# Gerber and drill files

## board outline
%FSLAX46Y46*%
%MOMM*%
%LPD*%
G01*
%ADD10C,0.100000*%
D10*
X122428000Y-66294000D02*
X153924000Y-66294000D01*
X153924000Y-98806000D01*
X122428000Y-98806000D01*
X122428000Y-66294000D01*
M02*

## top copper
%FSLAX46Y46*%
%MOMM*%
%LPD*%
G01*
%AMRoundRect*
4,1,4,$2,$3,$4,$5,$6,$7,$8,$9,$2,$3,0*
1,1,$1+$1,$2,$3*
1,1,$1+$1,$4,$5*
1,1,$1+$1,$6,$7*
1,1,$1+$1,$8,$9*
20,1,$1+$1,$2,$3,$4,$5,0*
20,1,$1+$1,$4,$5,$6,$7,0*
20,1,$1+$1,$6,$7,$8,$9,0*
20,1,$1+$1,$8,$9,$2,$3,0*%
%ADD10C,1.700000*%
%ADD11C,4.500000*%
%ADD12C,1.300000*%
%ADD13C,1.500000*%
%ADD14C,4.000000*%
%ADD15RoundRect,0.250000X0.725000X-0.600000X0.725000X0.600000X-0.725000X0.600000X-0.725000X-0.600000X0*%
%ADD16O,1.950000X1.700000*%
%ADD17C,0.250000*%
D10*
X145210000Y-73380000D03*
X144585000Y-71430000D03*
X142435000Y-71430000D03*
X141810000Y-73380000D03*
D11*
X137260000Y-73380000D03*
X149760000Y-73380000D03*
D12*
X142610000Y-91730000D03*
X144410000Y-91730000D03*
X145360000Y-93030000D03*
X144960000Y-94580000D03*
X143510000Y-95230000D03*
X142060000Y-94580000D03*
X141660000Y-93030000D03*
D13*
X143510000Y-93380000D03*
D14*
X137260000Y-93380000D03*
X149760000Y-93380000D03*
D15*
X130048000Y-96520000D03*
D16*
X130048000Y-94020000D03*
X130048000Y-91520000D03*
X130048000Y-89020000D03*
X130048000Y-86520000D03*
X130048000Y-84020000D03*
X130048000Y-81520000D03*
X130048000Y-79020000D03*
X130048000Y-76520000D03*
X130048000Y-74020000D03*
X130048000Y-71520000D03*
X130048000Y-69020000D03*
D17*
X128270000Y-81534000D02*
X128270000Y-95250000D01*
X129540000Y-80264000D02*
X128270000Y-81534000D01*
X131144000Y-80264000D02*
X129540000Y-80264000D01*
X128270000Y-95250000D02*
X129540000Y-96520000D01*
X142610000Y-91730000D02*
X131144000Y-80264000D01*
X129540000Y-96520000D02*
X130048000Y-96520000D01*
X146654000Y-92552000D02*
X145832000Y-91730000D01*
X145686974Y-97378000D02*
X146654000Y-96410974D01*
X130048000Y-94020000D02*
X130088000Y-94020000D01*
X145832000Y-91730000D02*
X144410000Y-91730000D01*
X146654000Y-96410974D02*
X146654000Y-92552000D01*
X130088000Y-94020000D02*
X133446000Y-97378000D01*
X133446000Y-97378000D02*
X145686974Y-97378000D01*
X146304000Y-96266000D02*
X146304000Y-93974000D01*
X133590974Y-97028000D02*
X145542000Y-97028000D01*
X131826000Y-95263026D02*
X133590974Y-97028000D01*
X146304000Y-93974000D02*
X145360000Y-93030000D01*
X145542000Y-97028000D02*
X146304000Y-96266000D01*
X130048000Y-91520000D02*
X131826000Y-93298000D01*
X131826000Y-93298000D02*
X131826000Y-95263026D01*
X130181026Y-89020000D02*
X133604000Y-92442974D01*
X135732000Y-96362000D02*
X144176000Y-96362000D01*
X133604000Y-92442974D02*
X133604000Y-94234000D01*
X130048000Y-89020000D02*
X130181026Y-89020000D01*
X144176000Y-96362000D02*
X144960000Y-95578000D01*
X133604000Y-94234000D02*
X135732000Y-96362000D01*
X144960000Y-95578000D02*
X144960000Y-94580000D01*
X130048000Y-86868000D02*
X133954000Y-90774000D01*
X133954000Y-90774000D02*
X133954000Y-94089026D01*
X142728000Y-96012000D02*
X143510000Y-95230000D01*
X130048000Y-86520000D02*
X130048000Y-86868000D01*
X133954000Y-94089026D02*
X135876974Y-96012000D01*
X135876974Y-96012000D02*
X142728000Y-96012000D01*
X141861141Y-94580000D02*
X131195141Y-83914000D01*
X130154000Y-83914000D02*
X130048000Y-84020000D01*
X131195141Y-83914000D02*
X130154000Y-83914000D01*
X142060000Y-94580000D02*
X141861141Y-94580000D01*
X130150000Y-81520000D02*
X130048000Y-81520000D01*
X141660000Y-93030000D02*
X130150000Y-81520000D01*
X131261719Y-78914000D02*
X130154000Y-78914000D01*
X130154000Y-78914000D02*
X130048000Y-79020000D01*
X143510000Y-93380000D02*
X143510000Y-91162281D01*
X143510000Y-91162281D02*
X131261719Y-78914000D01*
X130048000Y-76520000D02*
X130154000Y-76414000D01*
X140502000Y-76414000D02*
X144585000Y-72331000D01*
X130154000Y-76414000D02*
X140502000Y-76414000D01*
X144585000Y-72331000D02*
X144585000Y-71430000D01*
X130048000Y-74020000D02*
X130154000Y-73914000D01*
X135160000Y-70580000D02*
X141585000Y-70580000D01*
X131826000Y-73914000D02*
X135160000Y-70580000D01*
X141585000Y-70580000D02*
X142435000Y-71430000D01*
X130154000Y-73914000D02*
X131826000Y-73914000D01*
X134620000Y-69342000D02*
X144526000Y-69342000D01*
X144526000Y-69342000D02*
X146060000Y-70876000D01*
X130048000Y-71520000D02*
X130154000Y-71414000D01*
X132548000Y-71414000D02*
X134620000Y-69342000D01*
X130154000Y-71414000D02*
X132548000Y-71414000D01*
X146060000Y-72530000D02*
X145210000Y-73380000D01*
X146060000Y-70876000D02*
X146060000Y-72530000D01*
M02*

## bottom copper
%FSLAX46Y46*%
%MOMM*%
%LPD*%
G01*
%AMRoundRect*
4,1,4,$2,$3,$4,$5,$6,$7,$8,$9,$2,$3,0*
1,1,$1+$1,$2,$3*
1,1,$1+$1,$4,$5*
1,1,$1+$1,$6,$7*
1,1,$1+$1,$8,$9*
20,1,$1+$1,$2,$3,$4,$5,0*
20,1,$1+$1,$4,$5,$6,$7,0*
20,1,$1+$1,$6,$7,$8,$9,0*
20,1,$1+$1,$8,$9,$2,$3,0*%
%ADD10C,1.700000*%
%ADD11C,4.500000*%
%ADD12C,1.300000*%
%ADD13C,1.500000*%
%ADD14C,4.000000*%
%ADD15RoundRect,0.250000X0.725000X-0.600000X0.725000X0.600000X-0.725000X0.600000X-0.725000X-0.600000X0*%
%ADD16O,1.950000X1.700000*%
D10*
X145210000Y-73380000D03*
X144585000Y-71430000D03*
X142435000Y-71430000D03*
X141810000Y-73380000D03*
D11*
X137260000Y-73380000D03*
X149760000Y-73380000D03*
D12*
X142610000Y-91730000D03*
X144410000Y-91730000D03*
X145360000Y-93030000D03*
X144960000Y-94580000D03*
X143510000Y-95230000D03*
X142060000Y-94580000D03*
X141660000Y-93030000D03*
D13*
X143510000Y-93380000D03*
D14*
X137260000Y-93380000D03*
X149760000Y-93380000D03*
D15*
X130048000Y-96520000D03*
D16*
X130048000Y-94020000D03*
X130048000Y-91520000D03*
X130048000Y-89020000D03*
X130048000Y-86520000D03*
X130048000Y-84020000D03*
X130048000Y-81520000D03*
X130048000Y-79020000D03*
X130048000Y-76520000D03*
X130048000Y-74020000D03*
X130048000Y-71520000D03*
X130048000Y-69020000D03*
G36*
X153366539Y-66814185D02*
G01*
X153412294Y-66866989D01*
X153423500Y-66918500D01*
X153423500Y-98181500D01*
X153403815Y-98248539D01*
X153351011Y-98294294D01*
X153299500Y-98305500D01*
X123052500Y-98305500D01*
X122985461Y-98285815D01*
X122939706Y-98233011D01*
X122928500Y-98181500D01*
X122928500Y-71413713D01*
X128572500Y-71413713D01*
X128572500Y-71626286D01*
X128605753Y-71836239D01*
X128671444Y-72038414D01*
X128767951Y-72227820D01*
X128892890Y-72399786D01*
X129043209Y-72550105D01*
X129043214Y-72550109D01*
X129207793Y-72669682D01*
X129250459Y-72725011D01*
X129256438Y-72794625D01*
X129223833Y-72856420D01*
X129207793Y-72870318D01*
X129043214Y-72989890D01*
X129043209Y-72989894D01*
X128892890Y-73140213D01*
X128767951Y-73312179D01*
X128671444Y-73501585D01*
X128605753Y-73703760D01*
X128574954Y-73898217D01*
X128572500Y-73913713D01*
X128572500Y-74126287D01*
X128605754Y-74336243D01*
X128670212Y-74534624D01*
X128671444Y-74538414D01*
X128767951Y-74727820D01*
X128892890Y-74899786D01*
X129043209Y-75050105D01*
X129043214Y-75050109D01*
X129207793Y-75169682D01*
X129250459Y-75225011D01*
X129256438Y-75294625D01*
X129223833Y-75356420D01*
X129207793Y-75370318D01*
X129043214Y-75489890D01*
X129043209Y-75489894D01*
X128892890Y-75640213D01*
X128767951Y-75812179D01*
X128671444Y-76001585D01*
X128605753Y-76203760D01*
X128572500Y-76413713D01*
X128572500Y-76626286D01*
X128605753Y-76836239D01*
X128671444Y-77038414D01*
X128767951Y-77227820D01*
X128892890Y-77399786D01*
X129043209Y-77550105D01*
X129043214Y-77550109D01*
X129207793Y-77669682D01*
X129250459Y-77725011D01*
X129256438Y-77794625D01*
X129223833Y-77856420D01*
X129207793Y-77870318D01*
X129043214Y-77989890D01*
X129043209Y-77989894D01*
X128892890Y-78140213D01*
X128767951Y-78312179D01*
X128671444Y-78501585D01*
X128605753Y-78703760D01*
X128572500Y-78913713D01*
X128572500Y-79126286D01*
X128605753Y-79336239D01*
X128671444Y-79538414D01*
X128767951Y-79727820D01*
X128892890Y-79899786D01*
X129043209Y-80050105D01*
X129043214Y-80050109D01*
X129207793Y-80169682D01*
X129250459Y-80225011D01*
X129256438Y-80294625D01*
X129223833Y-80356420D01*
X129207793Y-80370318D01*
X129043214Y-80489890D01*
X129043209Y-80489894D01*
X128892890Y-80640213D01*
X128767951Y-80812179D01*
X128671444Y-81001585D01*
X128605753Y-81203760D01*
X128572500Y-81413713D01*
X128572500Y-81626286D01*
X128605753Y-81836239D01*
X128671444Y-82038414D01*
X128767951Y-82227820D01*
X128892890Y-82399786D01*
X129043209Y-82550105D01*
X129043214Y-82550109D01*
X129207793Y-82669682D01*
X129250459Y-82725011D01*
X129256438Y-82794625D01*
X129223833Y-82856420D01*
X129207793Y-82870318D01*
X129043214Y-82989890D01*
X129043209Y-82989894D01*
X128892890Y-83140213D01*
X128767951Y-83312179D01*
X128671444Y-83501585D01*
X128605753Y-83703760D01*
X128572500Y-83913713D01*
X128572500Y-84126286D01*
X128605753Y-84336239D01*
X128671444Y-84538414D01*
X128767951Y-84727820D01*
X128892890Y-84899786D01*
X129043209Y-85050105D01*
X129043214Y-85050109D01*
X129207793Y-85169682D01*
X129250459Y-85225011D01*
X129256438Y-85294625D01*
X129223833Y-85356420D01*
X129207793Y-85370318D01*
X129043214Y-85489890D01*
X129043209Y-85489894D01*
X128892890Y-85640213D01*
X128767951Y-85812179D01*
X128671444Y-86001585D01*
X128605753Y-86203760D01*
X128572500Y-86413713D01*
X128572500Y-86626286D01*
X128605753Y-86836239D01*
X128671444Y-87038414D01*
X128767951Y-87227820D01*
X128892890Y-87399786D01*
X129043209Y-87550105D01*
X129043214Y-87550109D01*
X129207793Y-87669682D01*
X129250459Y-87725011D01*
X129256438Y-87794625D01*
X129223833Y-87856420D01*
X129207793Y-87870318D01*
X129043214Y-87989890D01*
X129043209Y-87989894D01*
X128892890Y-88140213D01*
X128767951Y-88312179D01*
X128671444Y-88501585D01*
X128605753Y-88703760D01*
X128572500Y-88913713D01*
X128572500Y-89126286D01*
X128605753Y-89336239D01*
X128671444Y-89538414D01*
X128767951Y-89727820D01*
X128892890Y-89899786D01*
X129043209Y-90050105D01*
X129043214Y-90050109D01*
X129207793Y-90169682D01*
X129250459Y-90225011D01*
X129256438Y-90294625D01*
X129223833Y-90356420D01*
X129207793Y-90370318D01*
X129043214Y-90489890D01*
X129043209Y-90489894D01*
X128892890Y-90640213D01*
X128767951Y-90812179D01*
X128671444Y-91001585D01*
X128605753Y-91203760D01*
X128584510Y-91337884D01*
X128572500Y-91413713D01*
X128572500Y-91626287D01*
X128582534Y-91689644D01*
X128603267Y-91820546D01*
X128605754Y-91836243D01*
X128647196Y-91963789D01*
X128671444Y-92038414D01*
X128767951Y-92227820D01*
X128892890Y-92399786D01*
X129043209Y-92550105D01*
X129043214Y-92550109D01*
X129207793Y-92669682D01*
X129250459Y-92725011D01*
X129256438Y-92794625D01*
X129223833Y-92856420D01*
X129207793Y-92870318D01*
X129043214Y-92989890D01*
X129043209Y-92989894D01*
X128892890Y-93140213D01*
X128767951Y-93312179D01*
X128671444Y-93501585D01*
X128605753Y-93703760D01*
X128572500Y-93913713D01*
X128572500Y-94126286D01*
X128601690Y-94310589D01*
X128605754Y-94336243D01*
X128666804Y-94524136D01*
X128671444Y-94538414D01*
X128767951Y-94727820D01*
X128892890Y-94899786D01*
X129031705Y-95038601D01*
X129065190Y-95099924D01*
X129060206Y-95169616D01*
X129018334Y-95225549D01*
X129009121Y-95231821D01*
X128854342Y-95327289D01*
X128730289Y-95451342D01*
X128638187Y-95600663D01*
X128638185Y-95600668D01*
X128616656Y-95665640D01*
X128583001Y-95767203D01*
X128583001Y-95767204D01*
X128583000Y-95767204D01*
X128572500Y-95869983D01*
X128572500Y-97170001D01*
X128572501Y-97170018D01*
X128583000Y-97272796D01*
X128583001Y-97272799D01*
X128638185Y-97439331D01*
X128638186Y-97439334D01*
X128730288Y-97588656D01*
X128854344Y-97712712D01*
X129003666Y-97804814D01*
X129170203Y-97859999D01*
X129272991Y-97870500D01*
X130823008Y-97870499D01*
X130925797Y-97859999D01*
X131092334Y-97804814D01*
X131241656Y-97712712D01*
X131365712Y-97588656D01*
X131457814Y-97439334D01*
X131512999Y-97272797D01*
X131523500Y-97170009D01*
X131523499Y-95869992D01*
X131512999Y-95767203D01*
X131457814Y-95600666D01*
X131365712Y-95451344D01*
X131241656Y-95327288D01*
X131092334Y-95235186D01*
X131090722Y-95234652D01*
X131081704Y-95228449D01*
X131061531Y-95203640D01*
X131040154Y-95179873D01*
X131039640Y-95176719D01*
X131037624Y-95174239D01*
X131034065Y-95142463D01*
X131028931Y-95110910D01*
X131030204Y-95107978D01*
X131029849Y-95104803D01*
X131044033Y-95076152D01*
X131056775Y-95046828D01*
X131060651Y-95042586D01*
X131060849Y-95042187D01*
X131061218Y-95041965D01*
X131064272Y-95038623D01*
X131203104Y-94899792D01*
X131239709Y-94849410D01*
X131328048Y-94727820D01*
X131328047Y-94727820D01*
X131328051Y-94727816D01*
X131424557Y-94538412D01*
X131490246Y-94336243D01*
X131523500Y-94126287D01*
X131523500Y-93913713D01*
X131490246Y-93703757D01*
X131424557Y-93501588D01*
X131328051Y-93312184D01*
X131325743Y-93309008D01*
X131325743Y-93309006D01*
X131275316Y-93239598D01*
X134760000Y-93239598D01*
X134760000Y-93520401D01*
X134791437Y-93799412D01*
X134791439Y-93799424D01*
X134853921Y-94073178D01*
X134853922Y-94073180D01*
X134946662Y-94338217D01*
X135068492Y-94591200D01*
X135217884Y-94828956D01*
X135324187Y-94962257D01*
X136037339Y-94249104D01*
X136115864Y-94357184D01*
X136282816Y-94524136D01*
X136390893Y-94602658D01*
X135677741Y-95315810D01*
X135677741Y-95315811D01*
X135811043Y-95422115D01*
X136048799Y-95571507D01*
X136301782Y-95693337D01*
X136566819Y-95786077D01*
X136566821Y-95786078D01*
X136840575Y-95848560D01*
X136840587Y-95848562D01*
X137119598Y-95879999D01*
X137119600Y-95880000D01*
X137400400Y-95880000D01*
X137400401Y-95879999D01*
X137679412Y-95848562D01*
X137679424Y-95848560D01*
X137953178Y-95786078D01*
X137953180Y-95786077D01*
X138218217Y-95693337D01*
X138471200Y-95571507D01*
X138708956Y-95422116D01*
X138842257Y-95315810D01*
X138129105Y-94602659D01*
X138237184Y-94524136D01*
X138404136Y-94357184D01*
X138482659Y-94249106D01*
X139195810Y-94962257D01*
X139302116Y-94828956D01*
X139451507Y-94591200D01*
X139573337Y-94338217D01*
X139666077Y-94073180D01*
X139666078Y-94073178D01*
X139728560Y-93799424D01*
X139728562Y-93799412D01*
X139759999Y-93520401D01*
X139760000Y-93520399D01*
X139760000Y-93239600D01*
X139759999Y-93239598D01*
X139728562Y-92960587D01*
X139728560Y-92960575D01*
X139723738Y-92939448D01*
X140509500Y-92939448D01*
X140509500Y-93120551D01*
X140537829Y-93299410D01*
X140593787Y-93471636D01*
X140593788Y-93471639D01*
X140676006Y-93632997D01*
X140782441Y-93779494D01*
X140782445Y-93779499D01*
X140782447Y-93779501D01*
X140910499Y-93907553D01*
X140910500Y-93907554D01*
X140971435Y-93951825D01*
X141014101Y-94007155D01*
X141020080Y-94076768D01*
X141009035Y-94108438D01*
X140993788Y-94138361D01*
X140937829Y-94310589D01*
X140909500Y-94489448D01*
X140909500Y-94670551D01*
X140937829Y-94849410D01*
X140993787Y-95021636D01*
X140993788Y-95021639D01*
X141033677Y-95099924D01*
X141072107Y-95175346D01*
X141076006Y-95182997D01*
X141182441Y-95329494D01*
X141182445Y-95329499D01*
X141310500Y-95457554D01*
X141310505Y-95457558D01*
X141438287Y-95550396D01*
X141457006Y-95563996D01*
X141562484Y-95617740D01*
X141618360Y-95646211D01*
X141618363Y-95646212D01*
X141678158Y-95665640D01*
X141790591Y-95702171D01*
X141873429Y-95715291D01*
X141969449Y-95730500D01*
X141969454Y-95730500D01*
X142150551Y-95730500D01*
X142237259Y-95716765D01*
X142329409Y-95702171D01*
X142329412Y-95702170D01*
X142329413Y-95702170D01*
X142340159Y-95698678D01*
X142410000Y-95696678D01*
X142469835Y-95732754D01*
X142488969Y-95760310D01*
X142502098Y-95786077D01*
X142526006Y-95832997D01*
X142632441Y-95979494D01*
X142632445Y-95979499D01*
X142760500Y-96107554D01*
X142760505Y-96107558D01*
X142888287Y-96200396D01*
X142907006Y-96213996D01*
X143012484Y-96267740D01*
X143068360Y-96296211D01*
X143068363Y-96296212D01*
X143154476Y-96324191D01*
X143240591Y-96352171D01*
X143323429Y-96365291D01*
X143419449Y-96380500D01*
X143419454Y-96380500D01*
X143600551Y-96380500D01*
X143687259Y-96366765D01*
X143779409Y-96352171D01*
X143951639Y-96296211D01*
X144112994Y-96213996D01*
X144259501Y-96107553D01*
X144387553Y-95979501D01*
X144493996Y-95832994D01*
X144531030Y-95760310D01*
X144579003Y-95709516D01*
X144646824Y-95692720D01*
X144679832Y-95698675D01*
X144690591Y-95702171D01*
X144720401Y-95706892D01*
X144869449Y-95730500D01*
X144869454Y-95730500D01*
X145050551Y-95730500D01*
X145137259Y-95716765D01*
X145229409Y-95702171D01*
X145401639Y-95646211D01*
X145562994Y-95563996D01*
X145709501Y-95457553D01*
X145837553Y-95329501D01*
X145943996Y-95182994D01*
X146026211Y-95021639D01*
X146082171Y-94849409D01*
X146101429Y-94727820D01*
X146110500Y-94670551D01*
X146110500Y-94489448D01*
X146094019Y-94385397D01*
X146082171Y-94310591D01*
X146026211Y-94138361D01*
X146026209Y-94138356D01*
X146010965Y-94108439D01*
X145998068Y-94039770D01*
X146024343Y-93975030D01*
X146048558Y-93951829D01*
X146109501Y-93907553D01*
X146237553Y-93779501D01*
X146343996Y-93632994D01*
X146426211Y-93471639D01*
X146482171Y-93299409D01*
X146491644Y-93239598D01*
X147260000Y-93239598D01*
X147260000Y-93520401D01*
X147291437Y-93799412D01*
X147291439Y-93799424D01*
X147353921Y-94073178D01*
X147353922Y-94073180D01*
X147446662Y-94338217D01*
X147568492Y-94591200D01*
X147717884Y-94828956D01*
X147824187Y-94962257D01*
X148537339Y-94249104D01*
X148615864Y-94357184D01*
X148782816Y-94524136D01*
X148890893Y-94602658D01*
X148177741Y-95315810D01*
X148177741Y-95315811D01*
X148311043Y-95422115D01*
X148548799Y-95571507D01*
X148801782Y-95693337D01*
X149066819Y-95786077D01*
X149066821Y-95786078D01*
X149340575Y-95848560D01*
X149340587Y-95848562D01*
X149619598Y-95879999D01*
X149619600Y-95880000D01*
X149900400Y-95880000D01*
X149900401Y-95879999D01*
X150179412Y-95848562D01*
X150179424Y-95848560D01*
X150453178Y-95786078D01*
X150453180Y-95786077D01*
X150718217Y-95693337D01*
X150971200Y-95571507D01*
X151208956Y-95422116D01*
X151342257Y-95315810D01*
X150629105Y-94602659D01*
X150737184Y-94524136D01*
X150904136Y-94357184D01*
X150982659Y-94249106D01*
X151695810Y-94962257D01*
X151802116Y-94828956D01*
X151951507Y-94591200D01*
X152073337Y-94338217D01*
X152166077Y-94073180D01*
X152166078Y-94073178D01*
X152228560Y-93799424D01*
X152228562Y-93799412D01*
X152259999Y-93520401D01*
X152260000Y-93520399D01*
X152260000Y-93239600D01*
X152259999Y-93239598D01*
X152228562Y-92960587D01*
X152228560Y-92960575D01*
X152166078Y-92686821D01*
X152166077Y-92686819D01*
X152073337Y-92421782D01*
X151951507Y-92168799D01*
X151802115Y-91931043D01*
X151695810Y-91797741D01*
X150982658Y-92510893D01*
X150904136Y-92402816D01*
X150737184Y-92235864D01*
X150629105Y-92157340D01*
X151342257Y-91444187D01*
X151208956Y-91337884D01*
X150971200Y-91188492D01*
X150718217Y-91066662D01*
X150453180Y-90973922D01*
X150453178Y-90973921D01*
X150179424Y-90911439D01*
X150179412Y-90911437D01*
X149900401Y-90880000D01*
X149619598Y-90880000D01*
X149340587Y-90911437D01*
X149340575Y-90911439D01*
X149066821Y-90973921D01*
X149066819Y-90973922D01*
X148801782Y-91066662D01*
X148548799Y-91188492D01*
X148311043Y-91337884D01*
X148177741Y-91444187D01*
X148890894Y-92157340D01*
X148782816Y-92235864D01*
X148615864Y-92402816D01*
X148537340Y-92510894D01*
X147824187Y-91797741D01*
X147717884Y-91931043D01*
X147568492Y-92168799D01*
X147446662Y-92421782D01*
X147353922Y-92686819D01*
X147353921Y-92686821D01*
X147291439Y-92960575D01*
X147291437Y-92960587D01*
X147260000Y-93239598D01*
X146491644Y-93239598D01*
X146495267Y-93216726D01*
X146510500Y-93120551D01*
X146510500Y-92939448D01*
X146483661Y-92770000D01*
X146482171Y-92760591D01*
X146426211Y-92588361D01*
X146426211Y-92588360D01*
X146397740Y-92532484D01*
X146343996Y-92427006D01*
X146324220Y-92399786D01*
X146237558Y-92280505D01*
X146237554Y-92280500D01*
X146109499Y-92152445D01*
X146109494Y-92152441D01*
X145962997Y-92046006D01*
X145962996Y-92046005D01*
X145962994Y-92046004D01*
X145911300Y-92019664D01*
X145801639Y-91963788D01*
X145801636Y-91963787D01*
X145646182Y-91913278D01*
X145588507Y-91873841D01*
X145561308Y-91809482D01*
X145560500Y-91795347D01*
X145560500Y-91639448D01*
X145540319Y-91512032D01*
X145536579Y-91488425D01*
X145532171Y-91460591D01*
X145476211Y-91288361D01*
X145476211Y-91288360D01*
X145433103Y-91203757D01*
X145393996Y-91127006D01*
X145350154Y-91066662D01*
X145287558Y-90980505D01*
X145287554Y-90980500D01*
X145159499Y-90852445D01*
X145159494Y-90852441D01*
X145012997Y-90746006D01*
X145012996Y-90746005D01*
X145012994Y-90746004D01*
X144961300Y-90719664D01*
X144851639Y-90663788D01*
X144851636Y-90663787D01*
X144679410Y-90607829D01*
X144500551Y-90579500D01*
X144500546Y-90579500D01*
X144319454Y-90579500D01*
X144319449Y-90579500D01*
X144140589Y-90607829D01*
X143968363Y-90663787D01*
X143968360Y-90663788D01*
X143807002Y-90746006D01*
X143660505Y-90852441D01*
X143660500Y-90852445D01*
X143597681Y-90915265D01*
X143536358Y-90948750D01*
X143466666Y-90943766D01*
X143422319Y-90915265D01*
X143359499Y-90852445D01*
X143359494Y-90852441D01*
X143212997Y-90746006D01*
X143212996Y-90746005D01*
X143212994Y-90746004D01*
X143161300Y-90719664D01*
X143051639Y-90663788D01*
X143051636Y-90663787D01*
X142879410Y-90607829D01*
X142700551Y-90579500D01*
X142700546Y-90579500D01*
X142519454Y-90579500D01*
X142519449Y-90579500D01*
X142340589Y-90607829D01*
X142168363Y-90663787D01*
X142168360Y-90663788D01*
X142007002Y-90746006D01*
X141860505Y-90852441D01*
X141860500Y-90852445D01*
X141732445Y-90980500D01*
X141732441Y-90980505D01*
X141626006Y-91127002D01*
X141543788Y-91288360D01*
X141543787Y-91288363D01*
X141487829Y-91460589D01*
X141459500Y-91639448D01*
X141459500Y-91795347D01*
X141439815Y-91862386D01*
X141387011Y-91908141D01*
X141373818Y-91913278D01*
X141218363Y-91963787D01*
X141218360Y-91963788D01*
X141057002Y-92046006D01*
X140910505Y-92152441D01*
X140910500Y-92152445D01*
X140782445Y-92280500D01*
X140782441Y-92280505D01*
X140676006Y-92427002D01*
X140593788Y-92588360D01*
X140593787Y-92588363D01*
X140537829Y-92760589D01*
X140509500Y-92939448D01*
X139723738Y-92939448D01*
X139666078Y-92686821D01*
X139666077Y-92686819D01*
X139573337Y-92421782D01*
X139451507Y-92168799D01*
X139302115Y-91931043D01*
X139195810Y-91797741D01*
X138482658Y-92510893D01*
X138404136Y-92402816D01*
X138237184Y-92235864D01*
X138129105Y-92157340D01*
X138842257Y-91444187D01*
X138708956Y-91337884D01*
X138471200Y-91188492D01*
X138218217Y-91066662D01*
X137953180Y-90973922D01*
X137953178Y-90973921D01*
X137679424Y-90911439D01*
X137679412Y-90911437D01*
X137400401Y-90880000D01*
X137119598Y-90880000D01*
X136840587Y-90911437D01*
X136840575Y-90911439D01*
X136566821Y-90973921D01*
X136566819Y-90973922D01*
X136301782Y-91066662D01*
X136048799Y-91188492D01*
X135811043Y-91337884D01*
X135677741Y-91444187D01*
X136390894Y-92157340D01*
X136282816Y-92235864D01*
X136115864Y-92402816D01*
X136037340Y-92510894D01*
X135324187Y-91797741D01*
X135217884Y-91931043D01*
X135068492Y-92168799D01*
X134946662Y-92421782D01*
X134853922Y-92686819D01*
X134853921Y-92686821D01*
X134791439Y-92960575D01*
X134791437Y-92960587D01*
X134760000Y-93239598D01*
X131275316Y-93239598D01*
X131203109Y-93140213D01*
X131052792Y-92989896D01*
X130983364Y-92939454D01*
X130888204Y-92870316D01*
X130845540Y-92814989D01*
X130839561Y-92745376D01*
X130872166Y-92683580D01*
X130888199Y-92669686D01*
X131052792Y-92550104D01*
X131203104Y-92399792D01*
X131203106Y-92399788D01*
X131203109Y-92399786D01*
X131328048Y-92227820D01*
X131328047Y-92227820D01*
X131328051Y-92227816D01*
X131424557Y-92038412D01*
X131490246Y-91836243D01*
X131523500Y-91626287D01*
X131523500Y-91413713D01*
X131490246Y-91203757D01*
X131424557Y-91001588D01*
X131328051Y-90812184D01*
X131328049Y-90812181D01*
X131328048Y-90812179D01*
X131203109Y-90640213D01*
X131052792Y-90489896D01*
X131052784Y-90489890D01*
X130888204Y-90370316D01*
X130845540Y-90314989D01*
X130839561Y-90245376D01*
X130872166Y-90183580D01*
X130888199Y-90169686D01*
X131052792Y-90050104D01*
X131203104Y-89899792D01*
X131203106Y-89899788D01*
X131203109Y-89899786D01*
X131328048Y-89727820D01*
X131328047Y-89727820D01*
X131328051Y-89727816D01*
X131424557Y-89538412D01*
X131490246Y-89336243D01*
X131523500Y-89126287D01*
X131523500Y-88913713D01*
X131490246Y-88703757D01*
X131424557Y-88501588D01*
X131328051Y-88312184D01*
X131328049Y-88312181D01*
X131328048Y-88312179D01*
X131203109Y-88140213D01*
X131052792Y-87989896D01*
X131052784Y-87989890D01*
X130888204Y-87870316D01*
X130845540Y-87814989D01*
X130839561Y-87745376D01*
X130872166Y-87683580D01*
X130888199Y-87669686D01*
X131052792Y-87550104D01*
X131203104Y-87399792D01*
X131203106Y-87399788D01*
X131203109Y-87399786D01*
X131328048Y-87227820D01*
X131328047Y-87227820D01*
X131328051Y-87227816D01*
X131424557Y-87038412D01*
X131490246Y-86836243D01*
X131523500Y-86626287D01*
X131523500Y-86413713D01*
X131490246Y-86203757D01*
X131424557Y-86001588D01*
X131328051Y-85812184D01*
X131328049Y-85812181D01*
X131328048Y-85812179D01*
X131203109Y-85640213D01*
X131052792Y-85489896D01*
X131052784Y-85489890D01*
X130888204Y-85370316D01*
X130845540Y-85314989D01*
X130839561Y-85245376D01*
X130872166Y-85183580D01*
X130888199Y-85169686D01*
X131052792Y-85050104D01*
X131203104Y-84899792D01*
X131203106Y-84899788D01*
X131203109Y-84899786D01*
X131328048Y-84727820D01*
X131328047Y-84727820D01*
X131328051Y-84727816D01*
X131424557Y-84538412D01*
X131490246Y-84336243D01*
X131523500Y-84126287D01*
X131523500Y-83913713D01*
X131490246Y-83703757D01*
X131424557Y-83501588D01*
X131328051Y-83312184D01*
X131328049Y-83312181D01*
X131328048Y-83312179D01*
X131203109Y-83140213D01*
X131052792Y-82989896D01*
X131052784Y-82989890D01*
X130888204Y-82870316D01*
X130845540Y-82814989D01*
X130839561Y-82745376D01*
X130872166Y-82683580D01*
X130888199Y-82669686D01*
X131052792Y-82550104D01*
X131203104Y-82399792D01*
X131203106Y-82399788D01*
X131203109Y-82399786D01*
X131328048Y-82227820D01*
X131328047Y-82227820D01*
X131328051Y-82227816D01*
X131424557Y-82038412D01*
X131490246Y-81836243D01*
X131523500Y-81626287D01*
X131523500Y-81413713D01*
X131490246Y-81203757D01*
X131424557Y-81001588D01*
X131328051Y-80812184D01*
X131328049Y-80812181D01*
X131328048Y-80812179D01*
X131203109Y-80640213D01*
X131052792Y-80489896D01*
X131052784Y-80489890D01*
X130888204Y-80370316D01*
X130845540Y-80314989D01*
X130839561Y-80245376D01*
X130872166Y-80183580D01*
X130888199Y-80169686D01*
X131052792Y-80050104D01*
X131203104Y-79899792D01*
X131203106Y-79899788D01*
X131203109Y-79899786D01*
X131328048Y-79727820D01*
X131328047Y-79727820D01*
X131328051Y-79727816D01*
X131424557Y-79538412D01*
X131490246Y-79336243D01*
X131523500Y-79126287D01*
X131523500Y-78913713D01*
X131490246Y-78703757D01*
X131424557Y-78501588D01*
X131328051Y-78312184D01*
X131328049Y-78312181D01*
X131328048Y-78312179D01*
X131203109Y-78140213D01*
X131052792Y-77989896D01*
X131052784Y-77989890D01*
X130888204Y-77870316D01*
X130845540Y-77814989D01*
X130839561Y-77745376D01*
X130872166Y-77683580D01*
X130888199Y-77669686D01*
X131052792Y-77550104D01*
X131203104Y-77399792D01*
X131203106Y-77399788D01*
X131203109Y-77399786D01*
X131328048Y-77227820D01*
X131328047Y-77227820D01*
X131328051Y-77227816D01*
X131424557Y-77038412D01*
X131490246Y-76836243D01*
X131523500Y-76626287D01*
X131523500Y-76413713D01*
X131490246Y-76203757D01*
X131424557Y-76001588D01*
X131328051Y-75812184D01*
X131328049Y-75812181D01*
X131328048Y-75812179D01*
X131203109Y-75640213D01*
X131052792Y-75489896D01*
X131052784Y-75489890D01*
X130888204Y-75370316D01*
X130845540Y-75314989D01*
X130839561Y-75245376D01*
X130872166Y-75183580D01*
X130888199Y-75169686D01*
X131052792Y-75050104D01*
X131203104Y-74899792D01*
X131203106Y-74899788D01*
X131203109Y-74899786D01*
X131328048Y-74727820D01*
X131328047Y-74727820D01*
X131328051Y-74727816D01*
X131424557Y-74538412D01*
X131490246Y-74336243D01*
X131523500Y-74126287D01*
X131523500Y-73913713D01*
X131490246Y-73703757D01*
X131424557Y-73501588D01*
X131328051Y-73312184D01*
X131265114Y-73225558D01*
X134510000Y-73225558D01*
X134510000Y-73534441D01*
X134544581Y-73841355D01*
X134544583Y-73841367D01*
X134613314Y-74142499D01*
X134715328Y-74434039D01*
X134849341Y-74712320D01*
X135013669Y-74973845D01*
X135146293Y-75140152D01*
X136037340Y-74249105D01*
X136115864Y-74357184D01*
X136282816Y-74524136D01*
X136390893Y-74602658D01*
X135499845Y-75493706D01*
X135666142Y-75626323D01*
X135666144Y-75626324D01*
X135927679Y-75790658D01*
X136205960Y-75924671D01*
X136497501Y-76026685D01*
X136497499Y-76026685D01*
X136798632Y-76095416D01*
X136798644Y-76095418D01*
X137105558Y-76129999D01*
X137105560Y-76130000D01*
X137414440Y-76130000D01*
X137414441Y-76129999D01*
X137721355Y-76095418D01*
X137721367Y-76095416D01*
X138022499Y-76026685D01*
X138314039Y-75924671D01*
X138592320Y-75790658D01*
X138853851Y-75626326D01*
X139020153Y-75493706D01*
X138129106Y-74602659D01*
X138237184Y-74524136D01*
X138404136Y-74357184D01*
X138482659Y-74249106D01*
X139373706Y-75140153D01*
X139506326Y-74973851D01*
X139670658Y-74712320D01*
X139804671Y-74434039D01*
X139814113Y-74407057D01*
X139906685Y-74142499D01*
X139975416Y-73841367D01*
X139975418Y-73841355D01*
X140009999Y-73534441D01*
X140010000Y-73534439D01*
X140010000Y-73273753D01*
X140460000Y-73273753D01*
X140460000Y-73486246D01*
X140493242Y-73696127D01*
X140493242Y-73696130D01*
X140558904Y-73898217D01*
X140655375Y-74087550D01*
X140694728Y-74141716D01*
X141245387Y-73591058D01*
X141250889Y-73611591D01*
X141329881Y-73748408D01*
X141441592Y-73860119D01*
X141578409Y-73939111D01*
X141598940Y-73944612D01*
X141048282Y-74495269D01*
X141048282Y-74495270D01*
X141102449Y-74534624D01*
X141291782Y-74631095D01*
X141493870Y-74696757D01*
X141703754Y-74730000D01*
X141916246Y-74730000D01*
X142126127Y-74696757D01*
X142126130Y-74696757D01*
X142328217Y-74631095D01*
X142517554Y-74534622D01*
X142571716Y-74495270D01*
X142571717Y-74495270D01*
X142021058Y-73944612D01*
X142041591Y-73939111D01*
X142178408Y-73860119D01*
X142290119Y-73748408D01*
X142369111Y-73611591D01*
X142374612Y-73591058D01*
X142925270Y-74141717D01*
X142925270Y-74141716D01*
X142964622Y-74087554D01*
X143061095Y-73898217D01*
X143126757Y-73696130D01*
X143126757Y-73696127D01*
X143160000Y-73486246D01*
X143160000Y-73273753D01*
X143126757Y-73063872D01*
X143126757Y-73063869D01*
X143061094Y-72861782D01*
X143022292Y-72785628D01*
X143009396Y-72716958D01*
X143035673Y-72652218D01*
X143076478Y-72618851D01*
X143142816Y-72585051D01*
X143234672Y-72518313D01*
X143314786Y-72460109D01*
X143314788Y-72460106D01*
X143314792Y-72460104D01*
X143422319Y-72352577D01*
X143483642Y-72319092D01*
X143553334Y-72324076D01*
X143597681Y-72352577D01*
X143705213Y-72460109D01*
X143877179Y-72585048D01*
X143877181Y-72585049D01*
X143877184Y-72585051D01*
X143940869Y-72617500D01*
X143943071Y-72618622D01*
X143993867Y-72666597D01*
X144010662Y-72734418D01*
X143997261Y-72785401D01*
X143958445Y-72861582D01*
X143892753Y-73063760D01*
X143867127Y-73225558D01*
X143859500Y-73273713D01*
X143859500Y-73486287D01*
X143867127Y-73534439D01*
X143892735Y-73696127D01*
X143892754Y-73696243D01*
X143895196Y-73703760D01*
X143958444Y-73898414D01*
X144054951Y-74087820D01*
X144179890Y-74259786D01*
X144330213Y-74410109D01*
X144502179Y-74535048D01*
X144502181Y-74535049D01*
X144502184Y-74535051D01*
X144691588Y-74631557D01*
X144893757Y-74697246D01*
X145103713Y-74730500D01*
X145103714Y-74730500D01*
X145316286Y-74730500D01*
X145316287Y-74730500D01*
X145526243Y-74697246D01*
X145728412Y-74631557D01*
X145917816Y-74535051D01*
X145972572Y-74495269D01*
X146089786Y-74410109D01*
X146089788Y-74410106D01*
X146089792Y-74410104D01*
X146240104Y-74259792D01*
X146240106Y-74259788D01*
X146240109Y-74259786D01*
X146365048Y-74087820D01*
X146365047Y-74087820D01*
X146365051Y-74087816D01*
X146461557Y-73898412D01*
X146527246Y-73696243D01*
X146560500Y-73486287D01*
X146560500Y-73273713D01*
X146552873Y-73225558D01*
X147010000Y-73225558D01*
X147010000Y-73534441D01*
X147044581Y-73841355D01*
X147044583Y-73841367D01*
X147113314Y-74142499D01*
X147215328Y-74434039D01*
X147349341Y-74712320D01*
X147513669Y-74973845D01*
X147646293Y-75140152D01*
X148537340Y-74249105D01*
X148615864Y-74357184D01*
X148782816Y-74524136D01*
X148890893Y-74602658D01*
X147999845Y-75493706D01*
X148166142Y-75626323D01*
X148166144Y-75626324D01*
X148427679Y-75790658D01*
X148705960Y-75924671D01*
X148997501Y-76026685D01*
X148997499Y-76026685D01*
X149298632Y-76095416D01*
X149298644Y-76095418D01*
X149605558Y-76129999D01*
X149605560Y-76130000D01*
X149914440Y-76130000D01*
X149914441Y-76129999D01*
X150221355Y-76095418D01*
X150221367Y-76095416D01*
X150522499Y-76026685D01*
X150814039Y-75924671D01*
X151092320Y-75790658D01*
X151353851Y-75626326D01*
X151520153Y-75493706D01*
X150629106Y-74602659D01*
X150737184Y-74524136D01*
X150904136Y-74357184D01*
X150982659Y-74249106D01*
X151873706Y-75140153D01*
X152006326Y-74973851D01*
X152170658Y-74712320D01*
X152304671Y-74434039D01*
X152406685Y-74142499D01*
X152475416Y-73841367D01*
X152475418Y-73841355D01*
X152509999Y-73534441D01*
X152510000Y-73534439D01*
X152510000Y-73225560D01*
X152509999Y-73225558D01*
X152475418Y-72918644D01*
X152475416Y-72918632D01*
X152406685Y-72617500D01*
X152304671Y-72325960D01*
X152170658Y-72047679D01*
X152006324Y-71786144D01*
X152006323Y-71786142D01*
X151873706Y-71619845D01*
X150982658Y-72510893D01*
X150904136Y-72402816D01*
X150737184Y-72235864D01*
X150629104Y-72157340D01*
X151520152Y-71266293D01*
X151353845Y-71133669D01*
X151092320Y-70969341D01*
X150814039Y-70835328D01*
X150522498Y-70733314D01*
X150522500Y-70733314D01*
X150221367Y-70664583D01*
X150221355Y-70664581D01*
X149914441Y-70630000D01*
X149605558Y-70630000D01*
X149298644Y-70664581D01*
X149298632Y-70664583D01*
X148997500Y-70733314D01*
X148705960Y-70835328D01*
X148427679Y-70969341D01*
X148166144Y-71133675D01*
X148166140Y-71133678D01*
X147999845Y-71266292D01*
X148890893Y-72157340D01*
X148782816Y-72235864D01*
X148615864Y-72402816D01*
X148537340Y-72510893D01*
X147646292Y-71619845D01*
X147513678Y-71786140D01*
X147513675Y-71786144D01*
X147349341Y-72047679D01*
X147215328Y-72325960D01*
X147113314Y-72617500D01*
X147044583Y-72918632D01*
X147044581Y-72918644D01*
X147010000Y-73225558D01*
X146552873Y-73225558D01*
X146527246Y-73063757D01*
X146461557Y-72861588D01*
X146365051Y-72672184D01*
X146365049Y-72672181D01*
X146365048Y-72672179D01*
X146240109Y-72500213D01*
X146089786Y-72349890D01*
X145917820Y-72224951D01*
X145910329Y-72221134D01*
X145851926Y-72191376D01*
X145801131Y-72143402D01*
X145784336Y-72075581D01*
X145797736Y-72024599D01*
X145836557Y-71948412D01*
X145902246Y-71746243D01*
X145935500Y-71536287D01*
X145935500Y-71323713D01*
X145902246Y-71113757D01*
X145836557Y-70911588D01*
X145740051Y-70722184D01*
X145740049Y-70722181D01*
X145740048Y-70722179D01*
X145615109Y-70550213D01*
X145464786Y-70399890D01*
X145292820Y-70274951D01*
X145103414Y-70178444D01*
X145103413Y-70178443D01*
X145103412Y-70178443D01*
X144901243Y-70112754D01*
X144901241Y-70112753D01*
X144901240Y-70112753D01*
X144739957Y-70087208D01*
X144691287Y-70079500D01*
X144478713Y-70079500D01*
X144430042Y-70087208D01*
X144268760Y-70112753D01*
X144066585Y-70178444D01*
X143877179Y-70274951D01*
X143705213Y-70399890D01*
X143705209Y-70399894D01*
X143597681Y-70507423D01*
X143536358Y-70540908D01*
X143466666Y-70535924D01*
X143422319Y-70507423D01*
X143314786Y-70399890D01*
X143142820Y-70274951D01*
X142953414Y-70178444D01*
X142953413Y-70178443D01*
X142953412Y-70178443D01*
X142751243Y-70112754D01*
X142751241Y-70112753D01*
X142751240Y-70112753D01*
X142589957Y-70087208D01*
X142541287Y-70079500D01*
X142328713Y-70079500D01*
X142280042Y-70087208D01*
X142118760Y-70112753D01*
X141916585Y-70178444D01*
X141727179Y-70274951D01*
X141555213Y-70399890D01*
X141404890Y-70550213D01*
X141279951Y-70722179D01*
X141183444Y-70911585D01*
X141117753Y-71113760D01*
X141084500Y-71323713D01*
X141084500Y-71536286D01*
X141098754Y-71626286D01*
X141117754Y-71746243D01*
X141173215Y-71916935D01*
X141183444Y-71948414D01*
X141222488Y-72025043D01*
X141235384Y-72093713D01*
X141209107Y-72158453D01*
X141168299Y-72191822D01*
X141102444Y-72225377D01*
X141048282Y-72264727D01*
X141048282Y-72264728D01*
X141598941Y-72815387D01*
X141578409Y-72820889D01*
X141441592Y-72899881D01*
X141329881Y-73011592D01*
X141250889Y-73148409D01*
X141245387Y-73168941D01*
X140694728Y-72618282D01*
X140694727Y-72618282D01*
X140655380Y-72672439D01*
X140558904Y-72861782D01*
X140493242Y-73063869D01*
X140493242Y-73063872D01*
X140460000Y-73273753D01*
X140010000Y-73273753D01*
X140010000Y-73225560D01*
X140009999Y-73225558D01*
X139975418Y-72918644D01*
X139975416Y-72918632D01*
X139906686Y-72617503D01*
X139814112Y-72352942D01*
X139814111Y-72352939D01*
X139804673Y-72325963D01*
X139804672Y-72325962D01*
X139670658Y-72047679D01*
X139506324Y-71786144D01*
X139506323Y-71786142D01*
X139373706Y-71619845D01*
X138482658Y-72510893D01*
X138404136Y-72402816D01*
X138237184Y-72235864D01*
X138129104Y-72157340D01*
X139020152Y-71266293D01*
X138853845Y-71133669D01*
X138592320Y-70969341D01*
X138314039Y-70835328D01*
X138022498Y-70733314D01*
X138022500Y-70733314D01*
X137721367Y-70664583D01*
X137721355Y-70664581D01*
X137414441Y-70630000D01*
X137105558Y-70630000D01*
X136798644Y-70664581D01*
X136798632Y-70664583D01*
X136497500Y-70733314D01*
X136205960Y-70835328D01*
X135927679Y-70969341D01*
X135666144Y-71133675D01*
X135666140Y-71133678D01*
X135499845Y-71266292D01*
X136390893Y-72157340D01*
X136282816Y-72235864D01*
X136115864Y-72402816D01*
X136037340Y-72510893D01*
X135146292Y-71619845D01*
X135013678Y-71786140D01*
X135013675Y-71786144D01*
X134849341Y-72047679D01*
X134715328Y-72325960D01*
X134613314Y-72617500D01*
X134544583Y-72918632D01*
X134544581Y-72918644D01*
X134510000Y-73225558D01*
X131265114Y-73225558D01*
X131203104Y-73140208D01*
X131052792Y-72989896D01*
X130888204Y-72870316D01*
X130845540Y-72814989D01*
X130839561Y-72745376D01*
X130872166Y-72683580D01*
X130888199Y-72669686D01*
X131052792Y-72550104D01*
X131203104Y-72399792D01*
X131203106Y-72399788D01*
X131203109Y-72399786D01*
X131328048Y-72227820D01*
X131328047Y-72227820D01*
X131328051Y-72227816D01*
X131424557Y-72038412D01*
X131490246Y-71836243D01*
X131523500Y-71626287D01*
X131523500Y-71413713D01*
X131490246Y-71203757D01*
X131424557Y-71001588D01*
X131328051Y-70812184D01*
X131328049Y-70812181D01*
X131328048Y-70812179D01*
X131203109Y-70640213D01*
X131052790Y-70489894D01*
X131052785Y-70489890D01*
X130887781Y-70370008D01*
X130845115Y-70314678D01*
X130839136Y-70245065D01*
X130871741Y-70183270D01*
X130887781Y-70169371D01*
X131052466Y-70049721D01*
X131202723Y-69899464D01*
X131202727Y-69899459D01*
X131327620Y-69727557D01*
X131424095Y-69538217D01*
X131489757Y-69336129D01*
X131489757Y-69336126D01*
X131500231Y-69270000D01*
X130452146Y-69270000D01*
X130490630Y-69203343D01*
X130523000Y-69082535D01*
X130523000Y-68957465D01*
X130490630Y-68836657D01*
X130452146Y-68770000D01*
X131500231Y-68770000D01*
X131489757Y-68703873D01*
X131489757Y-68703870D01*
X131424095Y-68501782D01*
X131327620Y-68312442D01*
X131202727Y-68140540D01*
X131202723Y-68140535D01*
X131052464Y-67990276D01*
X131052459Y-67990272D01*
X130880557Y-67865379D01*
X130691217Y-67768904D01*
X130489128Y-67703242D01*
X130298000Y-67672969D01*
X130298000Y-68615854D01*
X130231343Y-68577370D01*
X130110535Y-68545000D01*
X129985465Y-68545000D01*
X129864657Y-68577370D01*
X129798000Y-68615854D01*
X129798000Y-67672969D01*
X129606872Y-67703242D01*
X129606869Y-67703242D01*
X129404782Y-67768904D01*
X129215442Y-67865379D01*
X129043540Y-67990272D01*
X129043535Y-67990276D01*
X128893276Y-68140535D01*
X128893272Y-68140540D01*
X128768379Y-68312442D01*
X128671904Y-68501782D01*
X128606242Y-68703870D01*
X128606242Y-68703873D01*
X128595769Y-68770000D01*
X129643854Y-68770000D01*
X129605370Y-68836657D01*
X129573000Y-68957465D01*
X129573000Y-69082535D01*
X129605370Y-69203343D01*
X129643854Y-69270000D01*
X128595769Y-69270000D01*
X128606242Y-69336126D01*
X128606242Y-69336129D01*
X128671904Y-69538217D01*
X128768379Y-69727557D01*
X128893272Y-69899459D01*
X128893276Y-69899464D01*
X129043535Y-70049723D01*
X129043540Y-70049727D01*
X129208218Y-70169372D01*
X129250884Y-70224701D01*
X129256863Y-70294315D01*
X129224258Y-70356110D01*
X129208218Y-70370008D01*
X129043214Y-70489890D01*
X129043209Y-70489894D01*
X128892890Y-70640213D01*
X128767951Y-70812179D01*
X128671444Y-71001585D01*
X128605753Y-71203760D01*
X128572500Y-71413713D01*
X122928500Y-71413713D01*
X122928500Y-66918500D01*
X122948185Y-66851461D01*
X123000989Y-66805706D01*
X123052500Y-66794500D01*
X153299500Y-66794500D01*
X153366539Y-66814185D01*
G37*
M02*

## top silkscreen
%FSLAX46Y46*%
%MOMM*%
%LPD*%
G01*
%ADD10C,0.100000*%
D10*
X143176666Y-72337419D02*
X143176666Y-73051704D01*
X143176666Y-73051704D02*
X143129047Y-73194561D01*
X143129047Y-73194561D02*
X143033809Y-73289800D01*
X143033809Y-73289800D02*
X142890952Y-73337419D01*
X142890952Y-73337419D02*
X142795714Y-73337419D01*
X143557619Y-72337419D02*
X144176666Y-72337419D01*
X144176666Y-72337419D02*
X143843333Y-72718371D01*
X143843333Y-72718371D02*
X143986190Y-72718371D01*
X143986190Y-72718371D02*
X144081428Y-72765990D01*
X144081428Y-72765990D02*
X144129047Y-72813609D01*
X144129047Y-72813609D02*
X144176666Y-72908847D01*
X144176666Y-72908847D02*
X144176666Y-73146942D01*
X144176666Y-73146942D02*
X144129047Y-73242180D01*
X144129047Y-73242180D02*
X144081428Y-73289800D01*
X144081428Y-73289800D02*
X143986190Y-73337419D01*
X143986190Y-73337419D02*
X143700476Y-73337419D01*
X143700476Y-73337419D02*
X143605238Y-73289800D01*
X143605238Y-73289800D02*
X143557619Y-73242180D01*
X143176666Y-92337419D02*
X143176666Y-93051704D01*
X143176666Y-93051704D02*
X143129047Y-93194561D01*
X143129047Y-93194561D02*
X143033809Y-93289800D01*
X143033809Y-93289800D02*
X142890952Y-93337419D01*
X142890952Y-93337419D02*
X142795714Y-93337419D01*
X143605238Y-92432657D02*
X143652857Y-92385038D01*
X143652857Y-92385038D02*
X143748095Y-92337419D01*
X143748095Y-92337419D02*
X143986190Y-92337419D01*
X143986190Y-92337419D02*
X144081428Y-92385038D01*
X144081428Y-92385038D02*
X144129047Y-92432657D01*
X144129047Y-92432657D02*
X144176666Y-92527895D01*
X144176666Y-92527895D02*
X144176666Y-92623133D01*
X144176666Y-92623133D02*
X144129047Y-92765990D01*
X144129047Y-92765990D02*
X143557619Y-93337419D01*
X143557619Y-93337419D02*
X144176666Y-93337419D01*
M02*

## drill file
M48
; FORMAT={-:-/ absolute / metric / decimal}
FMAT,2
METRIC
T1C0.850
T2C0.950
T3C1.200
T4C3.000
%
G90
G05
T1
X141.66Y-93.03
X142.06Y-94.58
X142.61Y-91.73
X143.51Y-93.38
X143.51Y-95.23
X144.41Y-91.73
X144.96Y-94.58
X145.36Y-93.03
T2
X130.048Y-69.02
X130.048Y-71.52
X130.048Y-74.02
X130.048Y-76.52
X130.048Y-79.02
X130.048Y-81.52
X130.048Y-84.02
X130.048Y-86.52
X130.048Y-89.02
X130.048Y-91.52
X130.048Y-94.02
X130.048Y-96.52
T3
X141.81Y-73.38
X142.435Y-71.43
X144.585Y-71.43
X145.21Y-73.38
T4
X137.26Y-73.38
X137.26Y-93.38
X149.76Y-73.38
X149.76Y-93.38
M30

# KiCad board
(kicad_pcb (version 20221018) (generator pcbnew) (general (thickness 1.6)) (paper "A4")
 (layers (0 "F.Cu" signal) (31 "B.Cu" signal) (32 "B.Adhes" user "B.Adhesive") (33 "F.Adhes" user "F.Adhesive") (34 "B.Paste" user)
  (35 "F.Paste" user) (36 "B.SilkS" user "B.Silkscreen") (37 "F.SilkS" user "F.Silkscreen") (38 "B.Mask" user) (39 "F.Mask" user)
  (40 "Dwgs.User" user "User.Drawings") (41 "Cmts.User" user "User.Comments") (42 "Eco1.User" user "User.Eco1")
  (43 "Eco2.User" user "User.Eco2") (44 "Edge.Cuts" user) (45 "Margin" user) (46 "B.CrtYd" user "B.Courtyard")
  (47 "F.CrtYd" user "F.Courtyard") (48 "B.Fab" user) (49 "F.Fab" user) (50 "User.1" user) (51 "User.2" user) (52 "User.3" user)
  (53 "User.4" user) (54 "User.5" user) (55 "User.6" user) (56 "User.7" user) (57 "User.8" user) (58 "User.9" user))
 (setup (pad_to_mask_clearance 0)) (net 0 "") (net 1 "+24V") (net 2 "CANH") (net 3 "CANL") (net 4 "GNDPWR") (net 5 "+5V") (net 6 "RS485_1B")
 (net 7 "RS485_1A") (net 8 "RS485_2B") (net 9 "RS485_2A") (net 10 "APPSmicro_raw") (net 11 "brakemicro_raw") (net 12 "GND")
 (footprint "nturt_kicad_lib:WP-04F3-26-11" (layer "F.Cu") (at 143.51 73.38)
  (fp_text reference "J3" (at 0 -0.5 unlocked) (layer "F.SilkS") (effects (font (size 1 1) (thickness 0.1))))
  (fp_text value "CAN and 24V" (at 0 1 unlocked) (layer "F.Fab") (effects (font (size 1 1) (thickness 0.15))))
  (pad "1" thru_hole circle (at 1.7 0) (size 1.7 1.7) (drill 1.2) (layers "*.Cu" "*.Mask") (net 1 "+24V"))
  (pad "2" thru_hole circle (at 1.075 -1.95) (size 1.7 1.7) (drill 1.2) (layers "*.Cu" "*.Mask") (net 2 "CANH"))
  (pad "3" thru_hole circle (at -1.075 -1.95) (size 1.7 1.7) (drill 1.2) (layers "*.Cu" "*.Mask") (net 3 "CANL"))
  (pad "4" thru_hole circle (at -1.7 0) (size 1.7 1.7) (drill 1.2) (layers "*.Cu" "*.Mask") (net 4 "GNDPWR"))
  (pad "5" thru_hole circle (at -6.25 0) (size 4.5 4.5) (drill 3) (layers "*.Cu" "*.Mask") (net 4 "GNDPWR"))
  (pad "5" thru_hole circle (at 6.25 0) (size 4.5 4.5) (drill 3) (layers "*.Cu" "*.Mask") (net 4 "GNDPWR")))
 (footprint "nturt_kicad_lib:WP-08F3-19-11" (layer "F.Cu") (at 143.51 93.38)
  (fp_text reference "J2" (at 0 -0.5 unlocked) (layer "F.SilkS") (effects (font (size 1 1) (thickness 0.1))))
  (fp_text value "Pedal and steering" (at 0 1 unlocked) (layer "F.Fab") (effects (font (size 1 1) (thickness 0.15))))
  (pad "1" thru_hole circle (at -0.9 -1.65) (size 1.3 1.3) (drill 0.85) (layers "*.Cu" "*.Mask") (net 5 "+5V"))
  (pad "2" thru_hole circle (at 0.9 -1.65) (size 1.3 1.3) (drill 0.85) (layers "*.Cu" "*.Mask") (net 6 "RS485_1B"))
  (pad "3" thru_hole circle (at 1.85 -0.35) (size 1.3 1.3) (drill 0.85) (layers "*.Cu" "*.Mask") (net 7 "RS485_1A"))
  (pad "4" thru_hole circle (at 1.45 1.2) (size 1.3 1.3) (drill 0.85) (layers "*.Cu" "*.Mask") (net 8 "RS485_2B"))
  (pad "5" thru_hole circle (at 0 1.85) (size 1.3 1.3) (drill 0.85) (layers "*.Cu" "*.Mask") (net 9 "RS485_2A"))
  (pad "6" thru_hole circle (at -1.45 1.2) (size 1.3 1.3) (drill 0.85) (layers "*.Cu" "*.Mask") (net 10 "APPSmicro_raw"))
  (pad "7" thru_hole circle (at -1.85 -0.35) (size 1.3 1.3) (drill 0.85) (layers "*.Cu" "*.Mask") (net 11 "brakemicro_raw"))
  (pad "8" thru_hole circle (at 0 0) (size 1.5 1.5) (drill 0.85) (layers "*.Cu" "*.Mask") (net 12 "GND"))
  (pad "9" thru_hole circle (at -6.25 0) (size 4 4) (drill 3) (layers "*.Cu" "*.Mask") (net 4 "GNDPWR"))
  (pad "9" thru_hole circle (at 6.25 0) (size 4 4) (drill 3) (layers "*.Cu" "*.Mask") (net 4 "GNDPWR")))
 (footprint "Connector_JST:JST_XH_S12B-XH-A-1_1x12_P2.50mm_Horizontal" (layer "B.Cu") (at 130.048 96.52 90)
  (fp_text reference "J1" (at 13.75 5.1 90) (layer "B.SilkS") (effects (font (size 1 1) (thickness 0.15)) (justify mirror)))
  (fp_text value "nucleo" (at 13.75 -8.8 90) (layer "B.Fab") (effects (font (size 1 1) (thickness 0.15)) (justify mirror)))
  (pad "1" thru_hole roundrect (at 0 0 90) (size 1.7 1.95) (drill 0.95) (layers "*.Cu" "*.Mask") (roundrect_rratio 0.147059) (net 5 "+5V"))
  (pad "2" thru_hole oval (at 2.5 0 90) (size 1.7 1.95) (drill 0.95) (layers "*.Cu" "*.Mask") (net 6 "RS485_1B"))
  (pad "3" thru_hole oval (at 5 0 90) (size 1.7 1.95) (drill 0.95) (layers "*.Cu" "*.Mask") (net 7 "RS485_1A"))
  (pad "4" thru_hole oval (at 7.5 0 90) (size 1.7 1.95) (drill 0.95) (layers "*.Cu" "*.Mask") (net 8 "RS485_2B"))
  (pad "5" thru_hole oval (at 10 0 90) (size 1.7 1.95) (drill 0.95) (layers "*.Cu" "*.Mask") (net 9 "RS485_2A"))
  (pad "6" thru_hole oval (at 12.5 0 90) (size 1.7 1.95) (drill 0.95) (layers "*.Cu" "*.Mask") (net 10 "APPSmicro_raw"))
  (pad "7" thru_hole oval (at 15 0 90) (size 1.7 1.95) (drill 0.95) (layers "*.Cu" "*.Mask") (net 11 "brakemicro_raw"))
  (pad "8" thru_hole oval (at 17.5 0 90) (size 1.7 1.95) (drill 0.95) (layers "*.Cu" "*.Mask") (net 12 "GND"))
  (pad "9" thru_hole oval (at 20 0 90) (size 1.7 1.95) (drill 0.95) (layers "*.Cu" "*.Mask") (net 2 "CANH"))
  (pad "10" thru_hole oval (at 22.5 0 90) (size 1.7 1.95) (drill 0.95) (layers "*.Cu" "*.Mask") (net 3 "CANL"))
  (pad "11" thru_hole oval (at 25 0 90) (size 1.7 1.95) (drill 0.95) (layers "*.Cu" "*.Mask") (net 1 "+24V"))
  (pad "12" thru_hole oval (at 27.5 0 90) (size 1.7 1.95) (drill 0.95) (layers "*.Cu" "*.Mask") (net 4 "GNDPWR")))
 (gr_rect (start 122.428 66.294) (end 153.924 98.806) (stroke (width 0.1) (type default)) (fill none) (layer "Edge.Cuts"))
 (segment (start 128.27 81.534) (end 128.27 95.25) (width 0.25) (layer "F.Cu") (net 5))
 (segment (start 129.54 80.264) (end 128.27 81.534) (width 0.25) (layer "F.Cu") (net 5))
 (segment (start 131.144 80.264) (end 129.54 80.264) (width 0.25) (layer "F.Cu") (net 5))
 (segment (start 128.27 95.25) (end 129.54 96.52) (width 0.25) (layer "F.Cu") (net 5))
 (segment (start 142.61 91.73) (end 131.144 80.264) (width 0.25) (layer "F.Cu") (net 5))
 (segment (start 129.54 96.52) (end 130.048 96.52) (width 0.25) (layer "F.Cu") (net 5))
 (segment (start 146.654 92.552) (end 145.832 91.73) (width 0.25) (layer "F.Cu") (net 6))
 (segment (start 145.686974 97.378) (end 146.654 96.410974) (width 0.25) (layer "F.Cu") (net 6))
 (segment (start 130.048 94.02) (end 130.088 94.02) (width 0.25) (layer "F.Cu") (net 6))
 (segment (start 145.832 91.73) (end 144.41 91.73) (width 0.25) (layer "F.Cu") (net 6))
 (segment (start 146.654 96.410974) (end 146.654 92.552) (width 0.25) (layer "F.Cu") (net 6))
 (segment (start 130.088 94.02) (end 133.446 97.378) (width 0.25) (layer "F.Cu") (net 6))
 (segment (start 133.446 97.378) (end 145.686974 97.378) (width 0.25) (layer "F.Cu") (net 6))
 (segment (start 146.304 96.266) (end 146.304 93.974) (width 0.25) (layer "F.Cu") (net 7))
 (segment (start 133.590974 97.028) (end 145.542 97.028) (width 0.25) (layer "F.Cu") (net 7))
 (segment (start 131.826 95.263026) (end 133.590974 97.028) (width 0.25) (layer "F.Cu") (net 7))
 (segment (start 146.304 93.974) (end 145.36 93.03) (width 0.25) (layer "F.Cu") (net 7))
 (segment (start 145.542 97.028) (end 146.304 96.266) (width 0.25) (layer "F.Cu") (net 7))
 (segment (start 130.048 91.52) (end 131.826 93.298) (width 0.25) (layer "F.Cu") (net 7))
 (segment (start 131.826 93.298) (end 131.826 95.263026) (width 0.25) (layer "F.Cu") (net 7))
 (segment (start 130.181026 89.02) (end 133.604 92.442974) (width 0.25) (layer "F.Cu") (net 8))
 (segment (start 135.732 96.362) (end 144.176 96.362) (width 0.25) (layer "F.Cu") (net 8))
 (segment (start 133.604 92.442974) (end 133.604 94.234) (width 0.25) (layer "F.Cu") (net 8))
 (segment (start 130.048 89.02) (end 130.181026 89.02) (width 0.25) (layer "F.Cu") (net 8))
 (segment (start 144.176 96.362) (end 144.96 95.578) (width 0.25) (layer "F.Cu") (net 8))
 (segment (start 133.604 94.234) (end 135.732 96.362) (width 0.25) (layer "F.Cu") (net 8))
 (segment (start 144.96 95.578) (end 144.96 94.58) (width 0.25) (layer "F.Cu") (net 8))
 (segment (start 130.048 86.868) (end 133.954 90.774) (width 0.25) (layer "F.Cu") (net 9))
 (segment (start 133.954 90.774) (end 133.954 94.089026) (width 0.25) (layer "F.Cu") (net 9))
 (segment (start 142.728 96.012) (end 143.51 95.23) (width 0.25) (layer "F.Cu") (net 9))
 (segment (start 130.048 86.52) (end 130.048 86.868) (width 0.25) (layer "F.Cu") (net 9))
 (segment (start 133.954 94.089026) (end 135.876974 96.012) (width 0.25) (layer "F.Cu") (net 9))
 (segment (start 135.876974 96.012) (end 142.728 96.012) (width 0.25) (layer "F.Cu") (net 9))
 (segment (start 141.861141 94.58) (end 131.195141 83.914) (width 0.25) (layer "F.Cu") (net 10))
 (segment (start 130.154 83.914) (end 130.048 84.02) (width 0.25) (layer "F.Cu") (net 10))
 (segment (start 131.195141 83.914) (end 130.154 83.914) (width 0.25) (layer "F.Cu") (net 10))
 (segment (start 142.06 94.58) (end 141.861141 94.58) (width 0.25) (layer "F.Cu") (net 10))
 (segment (start 130.15 81.52) (end 130.048 81.52) (width 0.25) (layer "F.Cu") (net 11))
 (segment (start 141.66 93.03) (end 130.15 81.52) (width 0.25) (layer "F.Cu") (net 11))
 (segment (start 131.261719 78.914) (end 130.154 78.914) (width 0.25) (layer "F.Cu") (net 12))
 (segment (start 130.154 78.914) (end 130.048 79.02) (width 0.25) (layer "F.Cu") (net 12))
 (segment (start 143.51 93.38) (end 143.51 91.162281) (width 0.25) (layer "F.Cu") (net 12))
 (segment (start 143.51 91.162281) (end 131.261719 78.914) (width 0.25) (layer "F.Cu") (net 12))
 (segment (start 130.048 76.52) (end 130.154 76.414) (width 0.25) (layer "F.Cu") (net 2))
 (segment (start 140.502 76.414) (end 144.585 72.331) (width 0.25) (layer "F.Cu") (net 2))
 (segment (start 130.154 76.414) (end 140.502 76.414) (width 0.25) (layer "F.Cu") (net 2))
 (segment (start 144.585 72.331) (end 144.585 71.43) (width 0.25) (layer "F.Cu") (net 2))
 (segment (start 130.048 74.02) (end 130.154 73.914) (width 0.25) (layer "F.Cu") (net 3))
 (segment (start 135.16 70.58) (end 141.585 70.58) (width 0.25) (layer "F.Cu") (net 3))
 (segment (start 131.826 73.914) (end 135.16 70.58) (width 0.25) (layer "F.Cu") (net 3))
 (segment (start 141.585 70.58) (end 142.435 71.43) (width 0.25) (layer "F.Cu") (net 3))
 (segment (start 130.154 73.914) (end 131.826 73.914) (width 0.25) (layer "F.Cu") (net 3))
 (segment (start 134.62 69.342) (end 144.526 69.342) (width 0.25) (layer "F.Cu") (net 1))
 (segment (start 144.526 69.342) (end 146.06 70.876) (width 0.25) (layer "F.Cu") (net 1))
 (segment (start 130.048 71.52) (end 130.154 71.414) (width 0.25) (layer "F.Cu") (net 1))
 (segment (start 132.548 71.414) (end 134.62 69.342) (width 0.25) (layer "F.Cu") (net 1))
 (segment (start 130.154 71.414) (end 132.548 71.414) (width 0.25) (layer "F.Cu") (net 1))
 (segment (start 146.06 72.53) (end 145.21 73.38) (width 0.25) (layer "F.Cu") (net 1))
 (segment (start 146.06 70.876) (end 146.06 72.53) (width 0.25) (layer "F.Cu") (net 1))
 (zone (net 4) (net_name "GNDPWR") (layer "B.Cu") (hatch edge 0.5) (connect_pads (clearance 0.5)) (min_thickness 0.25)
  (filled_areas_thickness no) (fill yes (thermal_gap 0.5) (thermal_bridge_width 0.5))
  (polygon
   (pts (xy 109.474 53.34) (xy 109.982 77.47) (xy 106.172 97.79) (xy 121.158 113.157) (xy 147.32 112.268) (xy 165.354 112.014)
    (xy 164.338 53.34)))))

